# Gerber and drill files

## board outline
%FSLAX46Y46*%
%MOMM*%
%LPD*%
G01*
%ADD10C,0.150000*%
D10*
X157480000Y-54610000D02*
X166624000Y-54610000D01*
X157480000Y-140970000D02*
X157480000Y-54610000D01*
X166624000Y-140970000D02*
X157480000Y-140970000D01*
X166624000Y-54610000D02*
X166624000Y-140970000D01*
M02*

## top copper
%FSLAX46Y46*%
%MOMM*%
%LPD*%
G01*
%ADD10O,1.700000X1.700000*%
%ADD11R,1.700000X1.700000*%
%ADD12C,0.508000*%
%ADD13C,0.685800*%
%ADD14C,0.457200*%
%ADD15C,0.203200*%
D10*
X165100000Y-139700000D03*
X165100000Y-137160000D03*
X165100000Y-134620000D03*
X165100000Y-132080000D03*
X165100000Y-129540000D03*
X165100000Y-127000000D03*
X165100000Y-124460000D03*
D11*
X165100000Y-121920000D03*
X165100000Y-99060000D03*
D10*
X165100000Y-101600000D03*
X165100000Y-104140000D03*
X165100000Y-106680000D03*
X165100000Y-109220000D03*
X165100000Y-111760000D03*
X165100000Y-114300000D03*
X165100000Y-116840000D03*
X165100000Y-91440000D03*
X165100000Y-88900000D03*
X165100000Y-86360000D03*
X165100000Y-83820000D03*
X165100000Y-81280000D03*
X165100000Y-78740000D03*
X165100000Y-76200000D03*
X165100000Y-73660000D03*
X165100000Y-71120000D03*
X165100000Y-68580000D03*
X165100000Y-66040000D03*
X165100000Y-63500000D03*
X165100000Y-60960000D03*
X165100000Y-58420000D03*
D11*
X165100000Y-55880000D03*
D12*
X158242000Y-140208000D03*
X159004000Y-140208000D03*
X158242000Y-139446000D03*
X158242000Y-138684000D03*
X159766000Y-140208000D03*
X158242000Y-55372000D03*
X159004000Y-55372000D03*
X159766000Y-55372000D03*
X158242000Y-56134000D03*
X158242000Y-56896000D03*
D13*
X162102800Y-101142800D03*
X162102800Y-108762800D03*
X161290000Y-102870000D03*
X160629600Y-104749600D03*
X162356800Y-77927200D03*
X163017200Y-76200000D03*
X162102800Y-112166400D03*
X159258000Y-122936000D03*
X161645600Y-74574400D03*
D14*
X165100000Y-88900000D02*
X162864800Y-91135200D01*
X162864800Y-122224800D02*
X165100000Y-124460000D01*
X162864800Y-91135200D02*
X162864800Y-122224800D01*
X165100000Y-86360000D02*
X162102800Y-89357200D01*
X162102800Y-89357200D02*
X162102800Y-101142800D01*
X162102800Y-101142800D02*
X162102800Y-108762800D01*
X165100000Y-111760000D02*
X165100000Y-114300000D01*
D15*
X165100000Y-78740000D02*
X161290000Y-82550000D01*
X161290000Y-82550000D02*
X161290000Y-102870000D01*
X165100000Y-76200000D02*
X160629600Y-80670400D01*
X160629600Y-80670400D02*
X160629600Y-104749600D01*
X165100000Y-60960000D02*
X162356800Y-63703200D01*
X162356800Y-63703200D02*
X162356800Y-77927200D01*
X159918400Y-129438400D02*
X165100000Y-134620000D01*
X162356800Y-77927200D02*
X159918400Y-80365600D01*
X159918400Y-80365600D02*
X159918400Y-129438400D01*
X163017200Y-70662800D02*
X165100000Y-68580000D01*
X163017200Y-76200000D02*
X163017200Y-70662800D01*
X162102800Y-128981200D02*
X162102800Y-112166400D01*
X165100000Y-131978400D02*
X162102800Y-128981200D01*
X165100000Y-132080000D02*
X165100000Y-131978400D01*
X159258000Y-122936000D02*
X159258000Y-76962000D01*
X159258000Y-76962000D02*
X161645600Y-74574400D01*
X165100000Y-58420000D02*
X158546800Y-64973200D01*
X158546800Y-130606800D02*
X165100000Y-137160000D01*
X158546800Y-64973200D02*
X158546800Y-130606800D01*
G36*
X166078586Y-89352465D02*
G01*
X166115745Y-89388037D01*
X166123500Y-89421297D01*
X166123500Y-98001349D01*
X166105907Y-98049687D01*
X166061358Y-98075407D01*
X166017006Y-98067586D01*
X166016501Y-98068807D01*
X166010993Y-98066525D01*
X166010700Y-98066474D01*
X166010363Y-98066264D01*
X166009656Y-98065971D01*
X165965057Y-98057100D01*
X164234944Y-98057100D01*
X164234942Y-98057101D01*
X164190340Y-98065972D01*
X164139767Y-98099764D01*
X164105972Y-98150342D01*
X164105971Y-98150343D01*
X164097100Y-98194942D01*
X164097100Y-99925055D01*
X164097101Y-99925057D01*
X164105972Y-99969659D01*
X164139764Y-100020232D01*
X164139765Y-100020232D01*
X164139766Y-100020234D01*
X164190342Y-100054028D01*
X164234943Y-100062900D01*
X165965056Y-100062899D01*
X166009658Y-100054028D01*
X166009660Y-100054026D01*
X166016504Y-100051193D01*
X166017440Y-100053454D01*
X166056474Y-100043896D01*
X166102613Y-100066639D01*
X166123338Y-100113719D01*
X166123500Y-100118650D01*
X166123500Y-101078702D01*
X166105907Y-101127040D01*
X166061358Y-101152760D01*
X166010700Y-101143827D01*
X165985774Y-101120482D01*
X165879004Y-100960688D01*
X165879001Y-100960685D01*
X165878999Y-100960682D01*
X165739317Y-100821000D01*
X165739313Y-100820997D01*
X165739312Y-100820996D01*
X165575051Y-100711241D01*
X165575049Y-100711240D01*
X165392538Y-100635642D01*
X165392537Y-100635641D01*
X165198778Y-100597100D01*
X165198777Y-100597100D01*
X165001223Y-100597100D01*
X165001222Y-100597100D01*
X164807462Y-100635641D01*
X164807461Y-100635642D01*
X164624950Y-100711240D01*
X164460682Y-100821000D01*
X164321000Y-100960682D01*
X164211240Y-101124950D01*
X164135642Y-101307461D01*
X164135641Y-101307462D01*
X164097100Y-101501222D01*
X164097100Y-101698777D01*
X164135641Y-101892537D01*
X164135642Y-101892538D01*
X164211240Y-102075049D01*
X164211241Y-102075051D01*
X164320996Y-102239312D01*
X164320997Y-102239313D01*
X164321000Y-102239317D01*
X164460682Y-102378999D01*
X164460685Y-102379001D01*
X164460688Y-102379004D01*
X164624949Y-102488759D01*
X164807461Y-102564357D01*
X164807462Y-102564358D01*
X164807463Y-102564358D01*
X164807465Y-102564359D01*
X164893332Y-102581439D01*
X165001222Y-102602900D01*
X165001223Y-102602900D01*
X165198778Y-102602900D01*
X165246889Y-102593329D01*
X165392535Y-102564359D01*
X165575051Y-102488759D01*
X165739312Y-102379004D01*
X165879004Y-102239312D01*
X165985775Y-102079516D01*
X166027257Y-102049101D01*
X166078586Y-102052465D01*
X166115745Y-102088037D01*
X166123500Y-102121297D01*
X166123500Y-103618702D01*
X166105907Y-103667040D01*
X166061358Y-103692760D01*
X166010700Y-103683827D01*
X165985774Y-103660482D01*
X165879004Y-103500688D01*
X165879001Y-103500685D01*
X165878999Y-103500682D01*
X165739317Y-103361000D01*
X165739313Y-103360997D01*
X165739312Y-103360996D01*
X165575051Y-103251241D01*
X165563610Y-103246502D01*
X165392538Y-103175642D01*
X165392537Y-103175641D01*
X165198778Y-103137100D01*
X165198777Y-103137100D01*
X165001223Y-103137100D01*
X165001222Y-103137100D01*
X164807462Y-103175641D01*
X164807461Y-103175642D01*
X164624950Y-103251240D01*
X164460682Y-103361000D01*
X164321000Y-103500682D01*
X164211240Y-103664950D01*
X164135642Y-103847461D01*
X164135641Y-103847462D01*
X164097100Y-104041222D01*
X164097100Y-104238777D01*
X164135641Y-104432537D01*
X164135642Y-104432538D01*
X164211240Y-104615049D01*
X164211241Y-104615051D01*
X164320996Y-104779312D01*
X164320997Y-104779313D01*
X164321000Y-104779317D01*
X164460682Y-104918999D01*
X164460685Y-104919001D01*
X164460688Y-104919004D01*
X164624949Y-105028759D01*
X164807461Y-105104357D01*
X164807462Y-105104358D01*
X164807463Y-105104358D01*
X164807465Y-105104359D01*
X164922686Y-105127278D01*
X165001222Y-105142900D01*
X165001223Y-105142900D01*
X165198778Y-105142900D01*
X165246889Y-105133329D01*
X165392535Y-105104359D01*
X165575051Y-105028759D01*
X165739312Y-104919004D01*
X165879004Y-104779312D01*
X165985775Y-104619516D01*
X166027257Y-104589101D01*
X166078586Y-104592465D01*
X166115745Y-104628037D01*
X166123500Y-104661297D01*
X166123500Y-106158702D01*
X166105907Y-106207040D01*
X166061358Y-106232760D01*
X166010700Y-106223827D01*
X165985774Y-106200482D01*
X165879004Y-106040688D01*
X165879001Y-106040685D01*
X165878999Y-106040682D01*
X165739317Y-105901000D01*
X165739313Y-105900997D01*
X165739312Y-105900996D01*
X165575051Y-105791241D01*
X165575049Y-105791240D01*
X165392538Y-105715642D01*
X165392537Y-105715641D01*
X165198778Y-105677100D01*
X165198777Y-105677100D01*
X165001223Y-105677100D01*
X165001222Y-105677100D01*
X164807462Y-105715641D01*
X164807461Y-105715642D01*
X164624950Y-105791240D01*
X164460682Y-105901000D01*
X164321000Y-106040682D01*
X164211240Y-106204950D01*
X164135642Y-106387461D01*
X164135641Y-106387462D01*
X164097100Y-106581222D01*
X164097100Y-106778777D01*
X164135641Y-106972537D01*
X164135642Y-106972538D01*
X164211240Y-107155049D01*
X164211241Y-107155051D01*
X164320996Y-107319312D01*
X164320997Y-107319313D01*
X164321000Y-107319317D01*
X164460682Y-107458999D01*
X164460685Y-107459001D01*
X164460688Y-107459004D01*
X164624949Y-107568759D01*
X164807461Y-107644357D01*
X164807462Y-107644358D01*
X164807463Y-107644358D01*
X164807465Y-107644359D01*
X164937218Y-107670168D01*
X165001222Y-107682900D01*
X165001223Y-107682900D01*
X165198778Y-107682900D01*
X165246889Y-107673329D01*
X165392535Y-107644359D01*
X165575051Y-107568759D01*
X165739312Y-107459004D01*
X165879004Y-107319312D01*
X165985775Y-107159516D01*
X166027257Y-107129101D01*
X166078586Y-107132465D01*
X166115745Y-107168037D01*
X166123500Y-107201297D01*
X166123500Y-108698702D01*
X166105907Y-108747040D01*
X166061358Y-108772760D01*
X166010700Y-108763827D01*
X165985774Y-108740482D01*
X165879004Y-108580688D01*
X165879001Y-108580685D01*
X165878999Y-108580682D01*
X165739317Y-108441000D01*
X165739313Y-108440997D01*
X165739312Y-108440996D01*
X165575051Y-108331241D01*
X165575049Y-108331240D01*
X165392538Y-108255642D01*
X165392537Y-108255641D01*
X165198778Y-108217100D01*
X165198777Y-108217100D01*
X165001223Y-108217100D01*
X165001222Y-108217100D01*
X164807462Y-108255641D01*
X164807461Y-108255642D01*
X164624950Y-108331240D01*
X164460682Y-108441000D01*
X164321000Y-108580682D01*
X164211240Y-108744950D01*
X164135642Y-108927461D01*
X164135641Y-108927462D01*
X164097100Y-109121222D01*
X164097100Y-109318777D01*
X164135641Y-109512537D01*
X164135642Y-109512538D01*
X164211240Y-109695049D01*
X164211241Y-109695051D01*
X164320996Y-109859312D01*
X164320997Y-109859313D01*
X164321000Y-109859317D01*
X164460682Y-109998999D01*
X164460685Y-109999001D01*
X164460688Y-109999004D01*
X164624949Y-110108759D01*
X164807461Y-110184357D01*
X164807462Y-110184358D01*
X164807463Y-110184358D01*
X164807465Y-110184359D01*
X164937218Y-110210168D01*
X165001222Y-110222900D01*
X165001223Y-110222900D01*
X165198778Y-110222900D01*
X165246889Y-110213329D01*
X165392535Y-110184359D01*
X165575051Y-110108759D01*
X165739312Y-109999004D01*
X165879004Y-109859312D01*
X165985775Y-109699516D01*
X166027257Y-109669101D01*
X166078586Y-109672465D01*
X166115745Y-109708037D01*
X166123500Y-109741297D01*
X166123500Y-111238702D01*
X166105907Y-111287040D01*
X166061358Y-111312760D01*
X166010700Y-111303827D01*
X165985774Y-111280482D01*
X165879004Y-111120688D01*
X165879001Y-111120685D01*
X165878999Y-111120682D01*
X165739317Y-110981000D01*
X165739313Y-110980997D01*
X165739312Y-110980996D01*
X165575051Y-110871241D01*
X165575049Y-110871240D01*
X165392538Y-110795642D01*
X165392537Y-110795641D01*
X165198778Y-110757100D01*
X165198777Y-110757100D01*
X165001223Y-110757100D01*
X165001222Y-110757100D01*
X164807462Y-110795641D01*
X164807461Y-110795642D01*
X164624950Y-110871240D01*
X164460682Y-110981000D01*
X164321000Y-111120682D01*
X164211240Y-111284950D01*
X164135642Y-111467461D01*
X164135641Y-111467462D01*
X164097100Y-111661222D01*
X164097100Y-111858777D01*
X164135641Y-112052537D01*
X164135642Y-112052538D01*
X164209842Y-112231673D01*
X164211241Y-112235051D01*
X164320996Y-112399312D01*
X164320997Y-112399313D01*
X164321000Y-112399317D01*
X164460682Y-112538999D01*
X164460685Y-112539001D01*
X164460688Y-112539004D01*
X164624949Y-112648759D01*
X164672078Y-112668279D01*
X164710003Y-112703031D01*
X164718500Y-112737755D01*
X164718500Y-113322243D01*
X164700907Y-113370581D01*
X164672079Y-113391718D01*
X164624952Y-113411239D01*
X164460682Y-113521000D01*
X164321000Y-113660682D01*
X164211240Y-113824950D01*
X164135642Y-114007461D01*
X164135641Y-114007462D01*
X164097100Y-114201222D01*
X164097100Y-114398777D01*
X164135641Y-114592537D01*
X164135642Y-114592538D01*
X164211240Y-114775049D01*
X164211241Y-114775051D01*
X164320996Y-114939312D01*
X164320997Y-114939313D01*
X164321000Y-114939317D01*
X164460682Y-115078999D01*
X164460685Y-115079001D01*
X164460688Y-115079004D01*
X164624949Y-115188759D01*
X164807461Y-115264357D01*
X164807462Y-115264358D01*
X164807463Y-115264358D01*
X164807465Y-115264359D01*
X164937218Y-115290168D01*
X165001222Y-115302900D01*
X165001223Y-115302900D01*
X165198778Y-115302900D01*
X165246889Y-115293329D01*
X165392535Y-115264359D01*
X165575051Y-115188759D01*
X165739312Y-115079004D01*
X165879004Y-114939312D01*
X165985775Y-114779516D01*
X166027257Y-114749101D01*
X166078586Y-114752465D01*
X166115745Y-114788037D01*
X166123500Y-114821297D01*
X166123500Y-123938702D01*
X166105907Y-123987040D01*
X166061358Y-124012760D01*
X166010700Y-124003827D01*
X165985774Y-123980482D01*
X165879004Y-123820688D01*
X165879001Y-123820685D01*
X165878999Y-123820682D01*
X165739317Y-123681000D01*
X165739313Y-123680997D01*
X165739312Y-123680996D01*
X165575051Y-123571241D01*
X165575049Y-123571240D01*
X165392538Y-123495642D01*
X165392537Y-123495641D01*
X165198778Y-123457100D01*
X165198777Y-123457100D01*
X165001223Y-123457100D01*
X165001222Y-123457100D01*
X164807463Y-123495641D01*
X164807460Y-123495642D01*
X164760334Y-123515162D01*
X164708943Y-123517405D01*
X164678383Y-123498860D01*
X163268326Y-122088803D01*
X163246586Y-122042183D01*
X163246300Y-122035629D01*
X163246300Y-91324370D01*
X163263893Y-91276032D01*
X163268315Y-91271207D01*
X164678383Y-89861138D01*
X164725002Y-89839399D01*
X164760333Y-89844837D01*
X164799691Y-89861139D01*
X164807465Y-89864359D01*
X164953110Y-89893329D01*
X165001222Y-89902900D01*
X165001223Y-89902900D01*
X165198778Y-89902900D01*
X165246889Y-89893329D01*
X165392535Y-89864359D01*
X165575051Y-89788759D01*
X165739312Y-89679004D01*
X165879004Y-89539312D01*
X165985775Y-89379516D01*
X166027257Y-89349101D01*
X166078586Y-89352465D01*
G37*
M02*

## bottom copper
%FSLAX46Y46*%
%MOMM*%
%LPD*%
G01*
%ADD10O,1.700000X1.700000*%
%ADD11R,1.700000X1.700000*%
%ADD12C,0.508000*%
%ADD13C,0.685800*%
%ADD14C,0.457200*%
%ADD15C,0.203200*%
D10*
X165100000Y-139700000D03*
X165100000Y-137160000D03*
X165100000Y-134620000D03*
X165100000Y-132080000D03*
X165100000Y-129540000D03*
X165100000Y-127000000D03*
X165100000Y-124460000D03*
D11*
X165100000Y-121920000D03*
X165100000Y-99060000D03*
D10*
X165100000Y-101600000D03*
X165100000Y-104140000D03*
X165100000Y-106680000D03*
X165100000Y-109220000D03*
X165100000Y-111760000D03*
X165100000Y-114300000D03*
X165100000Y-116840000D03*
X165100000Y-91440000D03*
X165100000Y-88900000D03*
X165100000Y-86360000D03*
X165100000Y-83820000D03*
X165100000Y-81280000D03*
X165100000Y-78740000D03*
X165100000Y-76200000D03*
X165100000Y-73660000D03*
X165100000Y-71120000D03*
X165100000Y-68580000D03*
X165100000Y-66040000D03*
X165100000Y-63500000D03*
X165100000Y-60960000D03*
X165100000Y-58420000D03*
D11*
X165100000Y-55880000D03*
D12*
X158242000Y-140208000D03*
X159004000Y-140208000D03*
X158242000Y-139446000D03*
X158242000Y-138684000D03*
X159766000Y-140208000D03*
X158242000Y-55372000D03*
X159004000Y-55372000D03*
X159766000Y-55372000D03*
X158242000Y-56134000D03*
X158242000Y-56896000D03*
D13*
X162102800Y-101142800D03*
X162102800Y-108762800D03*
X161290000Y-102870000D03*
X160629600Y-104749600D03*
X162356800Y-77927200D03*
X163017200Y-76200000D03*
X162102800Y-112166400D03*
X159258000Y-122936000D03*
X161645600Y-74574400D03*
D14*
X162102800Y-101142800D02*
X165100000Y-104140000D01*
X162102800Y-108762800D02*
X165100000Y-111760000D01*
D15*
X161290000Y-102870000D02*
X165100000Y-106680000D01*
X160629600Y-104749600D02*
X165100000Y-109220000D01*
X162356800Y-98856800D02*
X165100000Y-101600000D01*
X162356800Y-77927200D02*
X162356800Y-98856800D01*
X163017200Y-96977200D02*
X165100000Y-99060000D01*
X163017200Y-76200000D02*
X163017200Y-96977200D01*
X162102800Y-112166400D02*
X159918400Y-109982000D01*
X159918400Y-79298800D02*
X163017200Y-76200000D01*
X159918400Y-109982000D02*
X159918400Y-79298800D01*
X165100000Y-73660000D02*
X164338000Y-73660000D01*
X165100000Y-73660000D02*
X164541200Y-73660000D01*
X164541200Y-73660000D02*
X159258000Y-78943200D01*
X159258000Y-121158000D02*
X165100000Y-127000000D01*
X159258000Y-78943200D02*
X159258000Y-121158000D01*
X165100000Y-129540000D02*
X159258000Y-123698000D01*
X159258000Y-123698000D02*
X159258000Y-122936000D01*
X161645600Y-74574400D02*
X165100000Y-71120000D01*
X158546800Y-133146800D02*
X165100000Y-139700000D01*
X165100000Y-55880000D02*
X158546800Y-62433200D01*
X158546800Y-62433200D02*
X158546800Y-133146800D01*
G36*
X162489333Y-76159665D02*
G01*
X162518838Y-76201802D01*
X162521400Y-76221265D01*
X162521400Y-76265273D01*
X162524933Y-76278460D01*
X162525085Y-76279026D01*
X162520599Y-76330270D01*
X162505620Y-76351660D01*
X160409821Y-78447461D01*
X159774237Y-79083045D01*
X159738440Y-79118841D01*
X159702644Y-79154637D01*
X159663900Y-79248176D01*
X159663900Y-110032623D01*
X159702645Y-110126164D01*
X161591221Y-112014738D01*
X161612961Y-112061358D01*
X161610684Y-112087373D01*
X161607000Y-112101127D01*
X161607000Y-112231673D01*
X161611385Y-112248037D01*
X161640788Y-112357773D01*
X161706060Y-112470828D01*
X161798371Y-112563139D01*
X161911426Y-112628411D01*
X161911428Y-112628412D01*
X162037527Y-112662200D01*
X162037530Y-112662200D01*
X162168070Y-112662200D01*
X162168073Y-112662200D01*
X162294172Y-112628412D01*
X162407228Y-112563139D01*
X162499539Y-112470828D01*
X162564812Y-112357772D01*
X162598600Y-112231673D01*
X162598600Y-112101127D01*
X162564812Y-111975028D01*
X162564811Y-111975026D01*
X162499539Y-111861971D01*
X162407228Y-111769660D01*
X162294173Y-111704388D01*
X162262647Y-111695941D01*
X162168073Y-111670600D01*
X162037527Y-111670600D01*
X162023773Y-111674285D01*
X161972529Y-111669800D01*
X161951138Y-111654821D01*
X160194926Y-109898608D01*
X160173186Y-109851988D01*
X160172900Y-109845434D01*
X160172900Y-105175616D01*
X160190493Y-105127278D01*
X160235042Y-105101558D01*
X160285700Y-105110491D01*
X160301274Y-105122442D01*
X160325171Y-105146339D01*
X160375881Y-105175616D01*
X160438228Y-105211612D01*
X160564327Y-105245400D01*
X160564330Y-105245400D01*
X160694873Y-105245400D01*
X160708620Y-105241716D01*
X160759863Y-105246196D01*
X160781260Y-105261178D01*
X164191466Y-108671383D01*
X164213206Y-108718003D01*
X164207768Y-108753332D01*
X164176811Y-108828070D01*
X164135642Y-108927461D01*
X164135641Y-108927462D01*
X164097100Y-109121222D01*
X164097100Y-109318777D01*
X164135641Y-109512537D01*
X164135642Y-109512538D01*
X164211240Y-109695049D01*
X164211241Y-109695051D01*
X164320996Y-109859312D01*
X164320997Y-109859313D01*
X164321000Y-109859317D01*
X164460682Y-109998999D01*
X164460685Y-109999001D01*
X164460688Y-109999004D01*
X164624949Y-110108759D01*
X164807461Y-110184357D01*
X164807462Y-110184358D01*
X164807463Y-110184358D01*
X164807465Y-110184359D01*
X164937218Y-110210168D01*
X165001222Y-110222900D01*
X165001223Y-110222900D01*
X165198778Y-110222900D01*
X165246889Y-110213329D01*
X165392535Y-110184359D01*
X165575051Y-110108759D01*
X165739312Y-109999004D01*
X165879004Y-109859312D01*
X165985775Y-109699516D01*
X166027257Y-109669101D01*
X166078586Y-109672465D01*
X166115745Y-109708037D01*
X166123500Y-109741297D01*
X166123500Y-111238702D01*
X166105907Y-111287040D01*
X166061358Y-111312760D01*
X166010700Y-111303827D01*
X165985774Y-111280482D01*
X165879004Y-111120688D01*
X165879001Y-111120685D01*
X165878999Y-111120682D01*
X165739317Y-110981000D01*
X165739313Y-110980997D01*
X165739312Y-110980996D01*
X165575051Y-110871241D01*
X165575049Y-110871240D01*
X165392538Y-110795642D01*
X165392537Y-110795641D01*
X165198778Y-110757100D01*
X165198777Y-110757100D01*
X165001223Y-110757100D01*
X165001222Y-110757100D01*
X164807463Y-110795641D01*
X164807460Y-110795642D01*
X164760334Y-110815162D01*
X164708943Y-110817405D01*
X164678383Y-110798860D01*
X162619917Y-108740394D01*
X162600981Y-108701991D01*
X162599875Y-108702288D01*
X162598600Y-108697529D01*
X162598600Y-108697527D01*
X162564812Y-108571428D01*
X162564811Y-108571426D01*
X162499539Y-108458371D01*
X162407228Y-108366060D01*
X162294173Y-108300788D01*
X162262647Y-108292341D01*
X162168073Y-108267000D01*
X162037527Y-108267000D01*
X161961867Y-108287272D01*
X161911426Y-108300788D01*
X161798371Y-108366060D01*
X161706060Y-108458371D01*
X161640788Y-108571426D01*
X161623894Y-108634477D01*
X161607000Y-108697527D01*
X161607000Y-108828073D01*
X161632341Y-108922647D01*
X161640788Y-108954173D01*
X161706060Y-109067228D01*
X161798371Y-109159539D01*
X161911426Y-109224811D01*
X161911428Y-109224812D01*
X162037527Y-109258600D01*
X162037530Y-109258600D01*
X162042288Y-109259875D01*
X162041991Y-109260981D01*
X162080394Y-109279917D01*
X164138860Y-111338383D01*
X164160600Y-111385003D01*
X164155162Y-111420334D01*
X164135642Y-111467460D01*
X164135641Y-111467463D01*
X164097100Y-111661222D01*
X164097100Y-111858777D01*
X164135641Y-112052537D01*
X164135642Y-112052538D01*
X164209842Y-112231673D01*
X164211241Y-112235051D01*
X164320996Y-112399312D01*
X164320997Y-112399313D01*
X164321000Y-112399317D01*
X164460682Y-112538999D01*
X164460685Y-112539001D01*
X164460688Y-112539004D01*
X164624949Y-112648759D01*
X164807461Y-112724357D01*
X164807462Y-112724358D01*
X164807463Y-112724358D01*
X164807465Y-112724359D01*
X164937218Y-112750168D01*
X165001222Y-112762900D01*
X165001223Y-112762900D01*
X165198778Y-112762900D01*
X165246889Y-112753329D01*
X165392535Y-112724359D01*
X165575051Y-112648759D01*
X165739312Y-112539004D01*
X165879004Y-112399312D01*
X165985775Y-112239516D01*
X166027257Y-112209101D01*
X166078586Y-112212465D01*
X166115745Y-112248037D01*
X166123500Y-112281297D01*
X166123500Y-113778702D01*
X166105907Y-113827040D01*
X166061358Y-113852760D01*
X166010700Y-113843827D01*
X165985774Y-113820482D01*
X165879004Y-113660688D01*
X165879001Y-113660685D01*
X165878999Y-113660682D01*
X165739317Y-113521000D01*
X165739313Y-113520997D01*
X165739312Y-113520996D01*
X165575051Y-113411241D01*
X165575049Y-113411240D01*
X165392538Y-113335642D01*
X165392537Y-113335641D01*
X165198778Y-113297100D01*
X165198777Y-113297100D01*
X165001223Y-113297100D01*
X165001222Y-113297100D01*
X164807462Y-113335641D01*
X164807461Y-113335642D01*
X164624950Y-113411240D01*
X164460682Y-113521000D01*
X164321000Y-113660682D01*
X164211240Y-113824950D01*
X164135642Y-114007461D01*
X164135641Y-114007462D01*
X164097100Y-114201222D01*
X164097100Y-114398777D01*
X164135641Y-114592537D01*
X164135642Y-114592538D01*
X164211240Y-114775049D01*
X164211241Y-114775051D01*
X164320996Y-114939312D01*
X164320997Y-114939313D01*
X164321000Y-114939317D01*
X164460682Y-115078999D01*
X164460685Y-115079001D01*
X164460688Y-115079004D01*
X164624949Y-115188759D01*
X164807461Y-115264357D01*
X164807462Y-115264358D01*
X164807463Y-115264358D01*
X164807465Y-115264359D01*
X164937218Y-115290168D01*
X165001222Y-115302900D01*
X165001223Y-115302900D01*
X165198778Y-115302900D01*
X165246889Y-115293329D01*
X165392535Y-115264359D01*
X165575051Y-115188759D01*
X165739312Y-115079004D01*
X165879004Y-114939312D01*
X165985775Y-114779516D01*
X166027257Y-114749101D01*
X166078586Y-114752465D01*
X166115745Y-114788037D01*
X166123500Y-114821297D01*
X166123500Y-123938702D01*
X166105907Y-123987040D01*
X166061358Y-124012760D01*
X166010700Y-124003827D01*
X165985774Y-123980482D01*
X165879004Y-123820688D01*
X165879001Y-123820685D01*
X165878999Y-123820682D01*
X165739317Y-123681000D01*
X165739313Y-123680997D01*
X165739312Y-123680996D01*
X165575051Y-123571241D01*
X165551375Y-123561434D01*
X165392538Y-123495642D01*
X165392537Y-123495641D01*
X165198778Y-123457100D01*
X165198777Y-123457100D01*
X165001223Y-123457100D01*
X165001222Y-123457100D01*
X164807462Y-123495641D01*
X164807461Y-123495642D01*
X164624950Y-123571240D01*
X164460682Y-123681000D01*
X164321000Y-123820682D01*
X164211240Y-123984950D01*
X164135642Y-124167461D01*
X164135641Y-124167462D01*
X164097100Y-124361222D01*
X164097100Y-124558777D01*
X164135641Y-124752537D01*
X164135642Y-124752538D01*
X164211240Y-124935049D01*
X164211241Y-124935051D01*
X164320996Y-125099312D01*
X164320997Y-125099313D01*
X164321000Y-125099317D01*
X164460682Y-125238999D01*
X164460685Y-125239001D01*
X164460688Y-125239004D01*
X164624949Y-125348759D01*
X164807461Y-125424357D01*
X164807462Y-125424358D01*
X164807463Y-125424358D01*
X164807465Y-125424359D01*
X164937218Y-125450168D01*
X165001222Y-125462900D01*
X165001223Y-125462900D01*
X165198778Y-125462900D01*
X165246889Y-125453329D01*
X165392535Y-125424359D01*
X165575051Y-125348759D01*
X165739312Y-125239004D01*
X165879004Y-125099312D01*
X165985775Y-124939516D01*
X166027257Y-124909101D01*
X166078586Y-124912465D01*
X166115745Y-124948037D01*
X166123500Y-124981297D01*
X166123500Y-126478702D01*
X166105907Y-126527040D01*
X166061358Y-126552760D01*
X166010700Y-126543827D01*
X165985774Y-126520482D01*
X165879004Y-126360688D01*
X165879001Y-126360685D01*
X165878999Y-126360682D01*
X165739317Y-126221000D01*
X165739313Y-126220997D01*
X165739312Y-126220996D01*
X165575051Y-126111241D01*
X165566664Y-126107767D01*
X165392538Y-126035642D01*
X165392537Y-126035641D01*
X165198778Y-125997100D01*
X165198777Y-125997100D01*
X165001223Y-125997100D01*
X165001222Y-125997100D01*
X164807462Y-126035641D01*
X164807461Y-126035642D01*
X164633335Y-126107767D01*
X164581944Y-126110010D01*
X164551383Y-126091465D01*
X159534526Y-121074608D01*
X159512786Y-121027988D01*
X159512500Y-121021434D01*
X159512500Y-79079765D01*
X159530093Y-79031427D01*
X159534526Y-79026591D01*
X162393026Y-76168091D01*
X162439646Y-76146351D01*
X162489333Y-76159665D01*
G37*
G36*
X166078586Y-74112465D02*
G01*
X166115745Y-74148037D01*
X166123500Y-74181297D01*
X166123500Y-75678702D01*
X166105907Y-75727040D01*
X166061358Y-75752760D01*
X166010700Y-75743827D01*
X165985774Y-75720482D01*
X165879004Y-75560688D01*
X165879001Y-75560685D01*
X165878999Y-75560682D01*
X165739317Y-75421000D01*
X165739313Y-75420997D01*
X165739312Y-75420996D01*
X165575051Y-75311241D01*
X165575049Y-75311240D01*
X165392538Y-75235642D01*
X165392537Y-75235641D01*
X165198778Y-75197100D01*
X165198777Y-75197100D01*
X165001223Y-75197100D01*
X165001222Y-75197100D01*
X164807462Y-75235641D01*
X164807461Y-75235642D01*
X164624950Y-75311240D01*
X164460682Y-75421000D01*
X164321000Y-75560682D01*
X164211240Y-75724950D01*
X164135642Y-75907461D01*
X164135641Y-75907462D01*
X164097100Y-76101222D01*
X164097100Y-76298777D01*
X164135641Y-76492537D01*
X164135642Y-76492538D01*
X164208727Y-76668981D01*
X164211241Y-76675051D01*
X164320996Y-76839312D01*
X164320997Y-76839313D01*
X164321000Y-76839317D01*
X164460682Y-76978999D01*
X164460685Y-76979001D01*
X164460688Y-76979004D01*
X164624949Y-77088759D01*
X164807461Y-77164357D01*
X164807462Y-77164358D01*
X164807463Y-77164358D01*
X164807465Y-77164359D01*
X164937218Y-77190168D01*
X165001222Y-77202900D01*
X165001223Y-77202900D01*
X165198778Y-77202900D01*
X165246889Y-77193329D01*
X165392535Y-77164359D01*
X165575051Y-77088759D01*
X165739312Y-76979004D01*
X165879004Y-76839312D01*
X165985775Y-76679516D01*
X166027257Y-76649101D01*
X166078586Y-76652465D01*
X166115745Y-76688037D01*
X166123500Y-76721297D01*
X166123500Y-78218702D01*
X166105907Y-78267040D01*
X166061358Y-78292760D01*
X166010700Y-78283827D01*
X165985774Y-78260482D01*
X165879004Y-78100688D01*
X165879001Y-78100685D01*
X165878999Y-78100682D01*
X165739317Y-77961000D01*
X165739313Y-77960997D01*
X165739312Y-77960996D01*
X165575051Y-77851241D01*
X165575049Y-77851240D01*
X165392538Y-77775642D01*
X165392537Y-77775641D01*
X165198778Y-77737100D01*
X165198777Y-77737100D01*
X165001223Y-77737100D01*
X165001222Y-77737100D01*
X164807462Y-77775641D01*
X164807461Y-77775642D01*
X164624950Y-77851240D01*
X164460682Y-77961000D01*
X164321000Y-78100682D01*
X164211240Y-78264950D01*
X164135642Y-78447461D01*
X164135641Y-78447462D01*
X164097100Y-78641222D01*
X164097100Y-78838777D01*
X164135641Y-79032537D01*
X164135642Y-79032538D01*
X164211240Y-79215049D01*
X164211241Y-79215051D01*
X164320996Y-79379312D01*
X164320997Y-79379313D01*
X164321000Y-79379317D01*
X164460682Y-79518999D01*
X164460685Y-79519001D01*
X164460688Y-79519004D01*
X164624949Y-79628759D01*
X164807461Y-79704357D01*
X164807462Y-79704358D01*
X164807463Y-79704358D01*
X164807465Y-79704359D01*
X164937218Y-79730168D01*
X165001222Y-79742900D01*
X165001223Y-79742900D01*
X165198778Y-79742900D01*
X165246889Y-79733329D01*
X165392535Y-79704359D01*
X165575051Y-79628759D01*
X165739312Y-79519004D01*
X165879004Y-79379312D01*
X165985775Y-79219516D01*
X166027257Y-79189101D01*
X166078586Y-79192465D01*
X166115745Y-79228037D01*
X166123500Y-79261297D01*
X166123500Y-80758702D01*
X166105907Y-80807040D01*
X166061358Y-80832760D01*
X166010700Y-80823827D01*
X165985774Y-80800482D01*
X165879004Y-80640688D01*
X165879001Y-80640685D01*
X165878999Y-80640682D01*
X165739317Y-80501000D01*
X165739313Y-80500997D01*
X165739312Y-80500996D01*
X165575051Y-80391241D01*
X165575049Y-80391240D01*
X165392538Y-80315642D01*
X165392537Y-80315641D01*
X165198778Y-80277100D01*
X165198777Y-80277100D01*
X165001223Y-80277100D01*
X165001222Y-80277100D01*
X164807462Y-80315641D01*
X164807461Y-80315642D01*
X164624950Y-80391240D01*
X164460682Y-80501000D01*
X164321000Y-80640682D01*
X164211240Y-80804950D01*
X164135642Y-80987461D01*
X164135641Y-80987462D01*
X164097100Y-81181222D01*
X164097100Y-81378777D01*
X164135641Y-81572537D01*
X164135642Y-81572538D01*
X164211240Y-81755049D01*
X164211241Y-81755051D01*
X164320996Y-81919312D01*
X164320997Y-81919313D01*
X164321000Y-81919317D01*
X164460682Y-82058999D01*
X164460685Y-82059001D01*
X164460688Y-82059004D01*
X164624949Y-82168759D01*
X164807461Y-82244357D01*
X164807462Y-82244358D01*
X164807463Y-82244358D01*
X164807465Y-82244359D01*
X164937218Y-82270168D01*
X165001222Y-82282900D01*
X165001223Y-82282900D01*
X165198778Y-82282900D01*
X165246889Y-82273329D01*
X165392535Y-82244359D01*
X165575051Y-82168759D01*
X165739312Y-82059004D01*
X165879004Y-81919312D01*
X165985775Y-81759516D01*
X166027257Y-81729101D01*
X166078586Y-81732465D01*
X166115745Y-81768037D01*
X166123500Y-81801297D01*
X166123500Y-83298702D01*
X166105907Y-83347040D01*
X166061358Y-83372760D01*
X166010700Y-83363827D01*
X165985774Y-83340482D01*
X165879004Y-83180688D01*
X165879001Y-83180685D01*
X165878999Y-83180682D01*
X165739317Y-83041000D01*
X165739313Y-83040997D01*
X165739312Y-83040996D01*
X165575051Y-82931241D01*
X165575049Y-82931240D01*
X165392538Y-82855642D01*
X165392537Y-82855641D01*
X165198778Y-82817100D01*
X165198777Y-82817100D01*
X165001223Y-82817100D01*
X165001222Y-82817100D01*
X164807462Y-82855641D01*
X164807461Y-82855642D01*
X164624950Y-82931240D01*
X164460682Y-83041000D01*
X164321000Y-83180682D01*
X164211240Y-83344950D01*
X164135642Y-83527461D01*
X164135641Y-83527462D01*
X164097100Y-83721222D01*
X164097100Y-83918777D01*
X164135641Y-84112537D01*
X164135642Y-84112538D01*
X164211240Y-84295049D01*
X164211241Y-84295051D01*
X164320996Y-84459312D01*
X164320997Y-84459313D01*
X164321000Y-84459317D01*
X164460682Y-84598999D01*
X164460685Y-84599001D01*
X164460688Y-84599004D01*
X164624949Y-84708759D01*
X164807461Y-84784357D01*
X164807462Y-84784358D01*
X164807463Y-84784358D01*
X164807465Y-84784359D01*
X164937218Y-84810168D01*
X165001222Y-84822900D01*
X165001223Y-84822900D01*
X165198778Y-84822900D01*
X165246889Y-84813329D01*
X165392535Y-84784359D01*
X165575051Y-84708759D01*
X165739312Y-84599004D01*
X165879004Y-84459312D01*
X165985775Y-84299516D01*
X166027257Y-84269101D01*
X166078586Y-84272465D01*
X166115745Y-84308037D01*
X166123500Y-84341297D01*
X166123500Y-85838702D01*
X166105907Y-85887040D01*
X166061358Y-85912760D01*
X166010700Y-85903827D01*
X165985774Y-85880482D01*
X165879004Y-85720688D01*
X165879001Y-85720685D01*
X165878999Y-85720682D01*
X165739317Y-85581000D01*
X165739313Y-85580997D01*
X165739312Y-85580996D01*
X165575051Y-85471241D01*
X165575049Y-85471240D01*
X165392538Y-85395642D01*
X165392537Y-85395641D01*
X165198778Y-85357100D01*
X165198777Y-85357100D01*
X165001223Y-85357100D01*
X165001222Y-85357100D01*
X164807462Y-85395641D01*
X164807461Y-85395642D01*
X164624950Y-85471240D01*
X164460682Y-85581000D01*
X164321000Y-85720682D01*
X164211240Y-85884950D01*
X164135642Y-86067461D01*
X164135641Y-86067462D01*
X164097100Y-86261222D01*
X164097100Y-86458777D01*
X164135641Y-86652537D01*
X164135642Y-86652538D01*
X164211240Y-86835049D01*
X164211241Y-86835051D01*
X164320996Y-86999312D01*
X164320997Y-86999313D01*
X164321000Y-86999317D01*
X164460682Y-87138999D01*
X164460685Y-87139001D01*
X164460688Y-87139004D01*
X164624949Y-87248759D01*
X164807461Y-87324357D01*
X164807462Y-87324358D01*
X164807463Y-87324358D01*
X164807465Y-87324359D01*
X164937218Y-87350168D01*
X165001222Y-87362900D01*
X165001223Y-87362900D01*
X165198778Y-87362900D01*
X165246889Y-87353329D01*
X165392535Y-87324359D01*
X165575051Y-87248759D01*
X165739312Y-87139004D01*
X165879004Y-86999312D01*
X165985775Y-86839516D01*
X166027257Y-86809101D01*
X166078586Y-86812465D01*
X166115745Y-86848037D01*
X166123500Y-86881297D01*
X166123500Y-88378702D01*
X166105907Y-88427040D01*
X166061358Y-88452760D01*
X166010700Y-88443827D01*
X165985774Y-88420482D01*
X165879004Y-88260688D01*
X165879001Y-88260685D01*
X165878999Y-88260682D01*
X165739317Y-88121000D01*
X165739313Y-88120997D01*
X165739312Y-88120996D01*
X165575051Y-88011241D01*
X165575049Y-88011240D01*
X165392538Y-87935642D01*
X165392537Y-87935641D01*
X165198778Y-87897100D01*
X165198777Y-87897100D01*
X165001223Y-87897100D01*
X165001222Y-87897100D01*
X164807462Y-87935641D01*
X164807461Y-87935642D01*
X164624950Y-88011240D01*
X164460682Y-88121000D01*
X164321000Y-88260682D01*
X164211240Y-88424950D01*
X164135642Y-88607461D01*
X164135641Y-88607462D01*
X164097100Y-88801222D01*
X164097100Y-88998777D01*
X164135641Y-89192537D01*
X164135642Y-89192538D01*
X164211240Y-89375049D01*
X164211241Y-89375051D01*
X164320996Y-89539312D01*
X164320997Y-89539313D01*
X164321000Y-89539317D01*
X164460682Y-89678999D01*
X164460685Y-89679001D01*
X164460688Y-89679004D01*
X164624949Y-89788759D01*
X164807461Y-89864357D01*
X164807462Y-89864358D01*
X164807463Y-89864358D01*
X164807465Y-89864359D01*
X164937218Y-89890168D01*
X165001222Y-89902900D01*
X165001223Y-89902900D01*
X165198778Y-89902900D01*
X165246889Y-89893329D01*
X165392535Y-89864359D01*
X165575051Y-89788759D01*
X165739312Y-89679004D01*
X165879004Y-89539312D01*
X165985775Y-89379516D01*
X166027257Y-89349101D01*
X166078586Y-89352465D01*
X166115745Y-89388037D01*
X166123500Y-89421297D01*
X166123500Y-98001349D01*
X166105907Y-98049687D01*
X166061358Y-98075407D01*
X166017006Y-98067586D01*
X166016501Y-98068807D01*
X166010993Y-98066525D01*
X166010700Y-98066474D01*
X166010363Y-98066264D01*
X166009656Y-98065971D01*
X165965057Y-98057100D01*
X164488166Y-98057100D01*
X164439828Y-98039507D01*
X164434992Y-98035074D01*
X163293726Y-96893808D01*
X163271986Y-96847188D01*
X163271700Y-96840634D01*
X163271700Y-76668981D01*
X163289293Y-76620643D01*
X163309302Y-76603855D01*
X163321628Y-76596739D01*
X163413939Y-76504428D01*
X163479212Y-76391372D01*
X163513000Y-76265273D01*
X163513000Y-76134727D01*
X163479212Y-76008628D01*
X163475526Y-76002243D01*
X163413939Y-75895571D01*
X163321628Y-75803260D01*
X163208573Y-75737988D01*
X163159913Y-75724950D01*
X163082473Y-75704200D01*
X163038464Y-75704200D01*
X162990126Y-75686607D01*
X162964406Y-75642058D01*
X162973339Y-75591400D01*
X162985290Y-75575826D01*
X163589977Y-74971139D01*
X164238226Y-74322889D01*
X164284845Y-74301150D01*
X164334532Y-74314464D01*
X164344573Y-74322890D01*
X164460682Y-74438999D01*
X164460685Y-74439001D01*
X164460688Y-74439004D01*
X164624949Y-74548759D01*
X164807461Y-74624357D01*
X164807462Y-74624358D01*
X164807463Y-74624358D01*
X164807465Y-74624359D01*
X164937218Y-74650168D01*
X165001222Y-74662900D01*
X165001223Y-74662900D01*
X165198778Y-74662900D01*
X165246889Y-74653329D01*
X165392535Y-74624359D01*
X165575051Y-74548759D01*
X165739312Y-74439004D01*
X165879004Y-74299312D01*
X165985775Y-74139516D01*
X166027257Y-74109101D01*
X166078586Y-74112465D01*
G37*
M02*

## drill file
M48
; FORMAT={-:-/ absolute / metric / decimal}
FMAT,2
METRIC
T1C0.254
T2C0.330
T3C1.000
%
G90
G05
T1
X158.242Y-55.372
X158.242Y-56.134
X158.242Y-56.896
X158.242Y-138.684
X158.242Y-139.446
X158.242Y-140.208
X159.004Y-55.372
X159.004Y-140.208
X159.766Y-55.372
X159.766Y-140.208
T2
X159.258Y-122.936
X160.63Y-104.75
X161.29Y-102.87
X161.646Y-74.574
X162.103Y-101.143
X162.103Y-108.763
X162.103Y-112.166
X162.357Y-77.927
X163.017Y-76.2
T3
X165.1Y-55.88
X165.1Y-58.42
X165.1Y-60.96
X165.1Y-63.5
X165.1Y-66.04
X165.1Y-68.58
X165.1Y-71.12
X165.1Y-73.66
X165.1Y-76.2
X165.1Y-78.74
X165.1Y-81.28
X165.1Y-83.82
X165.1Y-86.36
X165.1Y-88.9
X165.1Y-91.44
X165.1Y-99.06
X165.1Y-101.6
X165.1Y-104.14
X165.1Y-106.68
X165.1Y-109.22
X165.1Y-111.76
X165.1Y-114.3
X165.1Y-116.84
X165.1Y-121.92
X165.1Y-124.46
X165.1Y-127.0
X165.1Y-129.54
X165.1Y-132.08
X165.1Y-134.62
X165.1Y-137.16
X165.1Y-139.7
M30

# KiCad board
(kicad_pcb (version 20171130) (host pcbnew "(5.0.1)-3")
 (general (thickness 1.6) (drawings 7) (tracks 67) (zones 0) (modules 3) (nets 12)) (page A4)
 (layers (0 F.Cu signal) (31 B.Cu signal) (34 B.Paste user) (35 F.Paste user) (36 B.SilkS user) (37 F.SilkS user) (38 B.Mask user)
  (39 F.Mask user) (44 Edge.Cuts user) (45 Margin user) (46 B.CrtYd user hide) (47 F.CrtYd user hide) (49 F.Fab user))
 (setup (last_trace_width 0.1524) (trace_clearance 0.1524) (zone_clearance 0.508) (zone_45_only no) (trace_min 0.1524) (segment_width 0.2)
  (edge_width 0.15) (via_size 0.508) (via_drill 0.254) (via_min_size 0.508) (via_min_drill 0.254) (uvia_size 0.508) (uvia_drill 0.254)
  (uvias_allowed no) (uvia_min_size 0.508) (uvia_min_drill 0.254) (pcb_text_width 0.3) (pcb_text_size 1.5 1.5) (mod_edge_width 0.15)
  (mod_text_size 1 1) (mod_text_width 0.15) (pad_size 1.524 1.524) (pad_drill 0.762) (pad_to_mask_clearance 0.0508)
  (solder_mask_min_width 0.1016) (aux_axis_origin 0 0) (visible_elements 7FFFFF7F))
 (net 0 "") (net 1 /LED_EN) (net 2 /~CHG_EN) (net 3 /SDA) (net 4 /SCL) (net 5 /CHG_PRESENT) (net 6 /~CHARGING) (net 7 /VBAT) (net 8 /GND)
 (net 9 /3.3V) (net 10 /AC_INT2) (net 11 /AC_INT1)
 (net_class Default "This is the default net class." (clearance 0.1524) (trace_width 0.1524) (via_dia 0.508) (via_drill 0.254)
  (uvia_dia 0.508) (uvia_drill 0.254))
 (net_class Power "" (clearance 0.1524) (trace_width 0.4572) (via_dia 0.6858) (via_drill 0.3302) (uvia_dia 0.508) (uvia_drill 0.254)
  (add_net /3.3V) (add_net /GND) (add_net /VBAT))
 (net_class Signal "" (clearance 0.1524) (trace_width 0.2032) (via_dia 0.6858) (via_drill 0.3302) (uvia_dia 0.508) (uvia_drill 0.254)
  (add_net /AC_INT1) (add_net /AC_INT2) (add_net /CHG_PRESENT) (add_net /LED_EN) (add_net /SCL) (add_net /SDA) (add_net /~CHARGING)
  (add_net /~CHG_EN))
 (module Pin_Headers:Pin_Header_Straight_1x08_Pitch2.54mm (layer F.Cu) (at 165.1 121.92)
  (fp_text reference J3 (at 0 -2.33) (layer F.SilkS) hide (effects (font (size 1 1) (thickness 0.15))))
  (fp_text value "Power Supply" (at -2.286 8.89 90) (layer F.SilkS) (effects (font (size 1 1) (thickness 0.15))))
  (pad 8 thru_hole oval (at 0 17.78) (size 1.7 1.7) (drill 1) (layers *.Cu *.Mask) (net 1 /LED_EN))
  (pad 7 thru_hole oval (at 0 15.24) (size 1.7 1.7) (drill 1) (layers *.Cu *.Mask) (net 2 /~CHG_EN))
  (pad 6 thru_hole oval (at 0 12.7) (size 1.7 1.7) (drill 1) (layers *.Cu *.Mask) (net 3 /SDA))
  (pad 5 thru_hole oval (at 0 10.16) (size 1.7 1.7) (drill 1) (layers *.Cu *.Mask) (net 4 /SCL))
  (pad 4 thru_hole oval (at 0 7.62) (size 1.7 1.7) (drill 1) (layers *.Cu *.Mask) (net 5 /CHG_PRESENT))
  (pad 3 thru_hole oval (at 0 5.08) (size 1.7 1.7) (drill 1) (layers *.Cu *.Mask) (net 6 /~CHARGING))
  (pad 2 thru_hole oval (at 0 2.54) (size 1.7 1.7) (drill 1) (layers *.Cu *.Mask) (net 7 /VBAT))
  (pad 1 thru_hole rect (at 0 0) (size 1.7 1.7) (drill 1) (layers *.Cu *.Mask) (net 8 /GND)))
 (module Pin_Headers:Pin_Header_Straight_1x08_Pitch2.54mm (layer F.Cu) (at 165.1 99.06)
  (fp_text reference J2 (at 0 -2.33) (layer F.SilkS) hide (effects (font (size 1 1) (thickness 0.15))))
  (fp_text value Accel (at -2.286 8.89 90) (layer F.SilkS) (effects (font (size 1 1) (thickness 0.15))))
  (pad 1 thru_hole rect (at 0 0) (size 1.7 1.7) (drill 1) (layers *.Cu *.Mask) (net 4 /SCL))
  (pad 2 thru_hole oval (at 0 2.54) (size 1.7 1.7) (drill 1) (layers *.Cu *.Mask) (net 3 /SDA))
  (pad 3 thru_hole oval (at 0 5.08) (size 1.7 1.7) (drill 1) (layers *.Cu *.Mask) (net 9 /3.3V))
  (pad 4 thru_hole oval (at 0 7.62) (size 1.7 1.7) (drill 1) (layers *.Cu *.Mask) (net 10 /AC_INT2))
  (pad 5 thru_hole oval (at 0 10.16) (size 1.7 1.7) (drill 1) (layers *.Cu *.Mask) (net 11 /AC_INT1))
  (pad 6 thru_hole oval (at 0 12.7) (size 1.7 1.7) (drill 1) (layers *.Cu *.Mask) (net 9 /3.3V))
  (pad 7 thru_hole oval (at 0 15.24) (size 1.7 1.7) (drill 1) (layers *.Cu *.Mask) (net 9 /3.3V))
  (pad 8 thru_hole oval (at 0 17.78) (size 1.7 1.7) (drill 1) (layers *.Cu *.Mask) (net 8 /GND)))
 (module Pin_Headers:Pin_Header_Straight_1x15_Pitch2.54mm (layer F.Cu) (at 165.1 55.88)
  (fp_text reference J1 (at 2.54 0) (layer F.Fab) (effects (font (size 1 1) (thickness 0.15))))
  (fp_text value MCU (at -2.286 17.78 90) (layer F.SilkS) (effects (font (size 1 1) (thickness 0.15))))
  (pad 15 thru_hole oval (at 0 35.56) (size 1.7 1.7) (drill 1) (layers *.Cu *.Mask) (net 8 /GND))
  (pad 14 thru_hole oval (at 0 33.02) (size 1.7 1.7) (drill 1) (layers *.Cu *.Mask) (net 7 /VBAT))
  (pad 13 thru_hole oval (at 0 30.48) (size 1.7 1.7) (drill 1) (layers *.Cu *.Mask) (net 9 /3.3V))
  (pad 12 thru_hole oval (at 0 27.94) (size 1.7 1.7) (drill 1) (layers *.Cu *.Mask))
  (pad 11 thru_hole oval (at 0 25.4) (size 1.7 1.7) (drill 1) (layers *.Cu *.Mask))
  (pad 10 thru_hole oval (at 0 22.86) (size 1.7 1.7) (drill 1) (layers *.Cu *.Mask) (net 10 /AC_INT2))
  (pad 9 thru_hole oval (at 0 20.32) (size 1.7 1.7) (drill 1) (layers *.Cu *.Mask) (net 11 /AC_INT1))
  (pad 8 thru_hole oval (at 0 17.78) (size 1.7 1.7) (drill 1) (layers *.Cu *.Mask) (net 6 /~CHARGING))
  (pad 7 thru_hole oval (at 0 15.24) (size 1.7 1.7) (drill 1) (layers *.Cu *.Mask) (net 5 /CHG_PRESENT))
  (pad 6 thru_hole oval (at 0 12.7) (size 1.7 1.7) (drill 1) (layers *.Cu *.Mask) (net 4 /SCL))
  (pad 5 thru_hole oval (at 0 10.16) (size 1.7 1.7) (drill 1) (layers *.Cu *.Mask))
  (pad 4 thru_hole oval (at 0 7.62) (size 1.7 1.7) (drill 1) (layers *.Cu *.Mask))
  (pad 3 thru_hole oval (at 0 5.08) (size 1.7 1.7) (drill 1) (layers *.Cu *.Mask) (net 3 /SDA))
  (pad 2 thru_hole oval (at 0 2.54) (size 1.7 1.7) (drill 1) (layers *.Cu *.Mask) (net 2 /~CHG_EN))
  (pad 1 thru_hole rect (at 0 0) (size 1.7 1.7) (drill 1) (layers *.Cu *.Mask) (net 1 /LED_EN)))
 (gr_line (start 157.48 54.61) (end 166.624 54.61) (layer Edge.Cuts) (width 0.15))
 (gr_line (start 157.48 140.97) (end 157.48 54.61) (layer Edge.Cuts) (width 0.15))
 (gr_line (start 166.624 140.97) (end 157.48 140.97) (layer Edge.Cuts) (width 0.15))
 (gr_line (start 166.624 54.61) (end 166.624 140.97) (layer Edge.Cuts) (width 0.15))
 (via (at 158.242 140.208) (size 0.508) (drill 0.254) (layers F.Cu B.Cu) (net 8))
 (via (at 159.004 140.208) (size 0.508) (drill 0.254) (layers F.Cu B.Cu) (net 8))
 (via (at 158.242 139.446) (size 0.508) (drill 0.254) (layers F.Cu B.Cu) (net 8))
 (via (at 158.242 138.684) (size 0.508) (drill 0.254) (layers F.Cu B.Cu) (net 8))
 (via (at 159.766 140.208) (size 0.508) (drill 0.254) (layers F.Cu B.Cu) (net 8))
 (via (at 158.242 55.372) (size 0.508) (drill 0.254) (layers F.Cu B.Cu) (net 8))
 (via (at 159.004 55.372) (size 0.508) (drill 0.254) (layers F.Cu B.Cu) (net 8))
 (via (at 159.766 55.372) (size 0.508) (drill 0.254) (layers F.Cu B.Cu) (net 8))
 (via (at 158.242 56.134) (size 0.508) (drill 0.254) (layers F.Cu B.Cu) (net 8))
 (via (at 158.242 56.896) (size 0.508) (drill 0.254) (layers F.Cu B.Cu) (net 8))
 (segment (start 165.1 88.9) (end 162.8648 91.1352) (width 0.4572) (layer F.Cu) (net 7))
 (segment (start 162.8648 122.2248) (end 165.1 124.46) (width 0.4572) (layer F.Cu) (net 7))
 (segment (start 162.8648 91.1352) (end 162.8648 122.2248) (width 0.4572) (layer F.Cu) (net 7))
 (via (at 162.1028 101.1428) (size 0.6858) (drill 0.3302) (layers F.Cu B.Cu) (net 9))
 (segment (start 165.1 86.36) (end 162.1028 89.3572) (width 0.4572) (layer F.Cu) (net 9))
 (segment (start 162.1028 89.3572) (end 162.1028 101.1428) (width 0.4572) (layer F.Cu) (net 9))
 (segment (start 162.1028 101.1428) (end 165.1 104.14) (width 0.4572) (layer B.Cu) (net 9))
 (via (at 162.1028 108.7628) (size 0.6858) (drill 0.3302) (layers F.Cu B.Cu) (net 9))
 (segment (start 162.1028 101.1428) (end 162.1028 108.7628) (width 0.4572) (layer F.Cu) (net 9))
 (segment (start 162.1028 108.7628) (end 165.1 111.76) (width 0.4572) (layer B.Cu) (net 9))
 (segment (start 165.1 111.76) (end 165.1 114.3) (width 0.4572) (layer F.Cu) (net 9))
 (via (at 161.29 102.87) (size 0.6858) (drill 0.3302) (layers F.Cu B.Cu) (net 10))
 (segment (start 165.1 78.74) (end 161.29 82.55) (width 0.2032) (layer F.Cu) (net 10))
 (segment (start 161.29 82.55) (end 161.29 102.87) (width 0.2032) (layer F.Cu) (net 10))
 (segment (start 161.29 102.87) (end 165.1 106.68) (width 0.2032) (layer B.Cu) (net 10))
 (via (at 160.6296 104.7496) (size 0.6858) (drill 0.3302) (layers F.Cu B.Cu) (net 11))
 (segment (start 165.1 76.2) (end 160.6296 80.6704) (width 0.2032) (layer F.Cu) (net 11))
 (segment (start 160.6296 80.6704) (end 160.6296 104.7496) (width 0.2032) (layer F.Cu) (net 11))
 (segment (start 160.6296 104.7496) (end 165.1 109.22) (width 0.2032) (layer B.Cu) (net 11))
 (segment (start 165.1 60.96) (end 162.3568 63.7032) (width 0.2032) (layer F.Cu) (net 3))
 (via (at 162.3568 77.9272) (size 0.6858) (drill 0.3302) (layers F.Cu B.Cu) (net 3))
 (segment (start 162.3568 63.7032) (end 162.3568 77.9272) (width 0.2032) (layer F.Cu) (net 3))
 (segment (start 162.3568 98.8568) (end 165.1 101.6) (width 0.2032) (layer B.Cu) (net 3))
 (segment (start 162.3568 77.9272) (end 162.3568 98.8568) (width 0.2032) (layer B.Cu) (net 3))
 (segment (start 159.9184 129.4384) (end 165.1 134.62) (width 0.2032) (layer F.Cu) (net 3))
 (segment (start 162.3568 77.9272) (end 159.9184 80.3656) (width 0.2032) (layer F.Cu) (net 3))
 (segment (start 159.9184 80.3656) (end 159.9184 129.4384) (width 0.2032) (layer F.Cu) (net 3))
 (via (at 163.0172 76.2) (size 0.6858) (drill 0.3302) (layers F.Cu B.Cu) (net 4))
 (segment (start 163.0172 70.6628) (end 165.1 68.58) (width 0.2032) (layer F.Cu) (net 4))
 (segment (start 163.0172 76.2) (end 163.0172 70.6628) (width 0.2032) (layer F.Cu) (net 4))
 (segment (start 163.0172 96.9772) (end 165.1 99.06) (width 0.2032) (layer B.Cu) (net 4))
 (segment (start 163.0172 76.2) (end 163.0172 96.9772) (width 0.2032) (layer B.Cu) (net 4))
 (via (at 162.1028 112.1664) (size 0.6858) (drill 0.3302) (layers F.Cu B.Cu) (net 4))
 (segment (start 162.1028 128.9812) (end 162.1028 112.1664) (width 0.2032) (layer F.Cu) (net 4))
 (segment (start 162.1028 112.1664) (end 159.9184 109.982) (width 0.2032) (layer B.Cu) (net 4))
 (segment (start 159.9184 79.2988) (end 163.0172 76.2) (width 0.2032) (layer B.Cu) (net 4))
 (segment (start 159.9184 109.982) (end 159.9184 79.2988) (width 0.2032) (layer B.Cu) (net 4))
 (segment (start 165.1 131.9784) (end 162.1028 128.9812) (width 0.2032) (layer F.Cu) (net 4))
 (segment (start 165.1 132.08) (end 165.1 131.9784) (width 0.2032) (layer F.Cu) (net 4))
 (segment (start 165.1 73.66) (end 164.338 73.66) (width 0.2032) (layer B.Cu) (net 6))
 (segment (start 165.1 73.66) (end 164.5412 73.66) (width 0.2032) (layer B.Cu) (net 6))
 (segment (start 164.5412 73.66) (end 159.258 78.9432) (width 0.2032) (layer B.Cu) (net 6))
 (segment (start 159.258 121.158) (end 165.1 127) (width 0.2032) (layer B.Cu) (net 6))
 (segment (start 159.258 78.9432) (end 159.258 121.158) (width 0.2032) (layer B.Cu) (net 6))
 (via (at 159.258 122.936) (size 0.6858) (drill 0.3302) (layers F.Cu B.Cu) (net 5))
 (segment (start 165.1 129.54) (end 159.258 123.698) (width 0.2032) (layer B.Cu) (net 5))
 (segment (start 159.258 123.698) (end 159.258 122.936) (width 0.2032) (layer B.Cu) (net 5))
 (via (at 161.6456 74.5744) (size 0.6858) (drill 0.3302) (layers F.Cu B.Cu) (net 5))
 (segment (start 159.258 122.936) (end 159.258 76.962) (width 0.2032) (layer F.Cu) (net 5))
 (segment (start 159.258 76.962) (end 161.6456 74.5744) (width 0.2032) (layer F.Cu) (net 5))
 (segment (start 161.6456 74.5744) (end 165.1 71.12) (width 0.2032) (layer B.Cu) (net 5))
 (segment (start 165.1 58.42) (end 158.5468 64.9732) (width 0.2032) (layer F.Cu) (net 2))
 (segment (start 158.5468 130.6068) (end 165.1 137.16) (width 0.2032) (layer F.Cu) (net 2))
 (segment (start 158.5468 64.9732) (end 158.5468 130.6068) (width 0.2032) (layer F.Cu) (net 2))
 (segment (start 158.5468 133.1468) (end 165.1 139.7) (width 0.2032) (layer B.Cu) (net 1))
 (segment (start 165.1 55.88) (end 158.5468 62.4332) (width 0.2032) (layer B.Cu) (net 1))
 (segment (start 158.5468 62.4332) (end 158.5468 133.1468) (width 0.2032) (layer B.Cu) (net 1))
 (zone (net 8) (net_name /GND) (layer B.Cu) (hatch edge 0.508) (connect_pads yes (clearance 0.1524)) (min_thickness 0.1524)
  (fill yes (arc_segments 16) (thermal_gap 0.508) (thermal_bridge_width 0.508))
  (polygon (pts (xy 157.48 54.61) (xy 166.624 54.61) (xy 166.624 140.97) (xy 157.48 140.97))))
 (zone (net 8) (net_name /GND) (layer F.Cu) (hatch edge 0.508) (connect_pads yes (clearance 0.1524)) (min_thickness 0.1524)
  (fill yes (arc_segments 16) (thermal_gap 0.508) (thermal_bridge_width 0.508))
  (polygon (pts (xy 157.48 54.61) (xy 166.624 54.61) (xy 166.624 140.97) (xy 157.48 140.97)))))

